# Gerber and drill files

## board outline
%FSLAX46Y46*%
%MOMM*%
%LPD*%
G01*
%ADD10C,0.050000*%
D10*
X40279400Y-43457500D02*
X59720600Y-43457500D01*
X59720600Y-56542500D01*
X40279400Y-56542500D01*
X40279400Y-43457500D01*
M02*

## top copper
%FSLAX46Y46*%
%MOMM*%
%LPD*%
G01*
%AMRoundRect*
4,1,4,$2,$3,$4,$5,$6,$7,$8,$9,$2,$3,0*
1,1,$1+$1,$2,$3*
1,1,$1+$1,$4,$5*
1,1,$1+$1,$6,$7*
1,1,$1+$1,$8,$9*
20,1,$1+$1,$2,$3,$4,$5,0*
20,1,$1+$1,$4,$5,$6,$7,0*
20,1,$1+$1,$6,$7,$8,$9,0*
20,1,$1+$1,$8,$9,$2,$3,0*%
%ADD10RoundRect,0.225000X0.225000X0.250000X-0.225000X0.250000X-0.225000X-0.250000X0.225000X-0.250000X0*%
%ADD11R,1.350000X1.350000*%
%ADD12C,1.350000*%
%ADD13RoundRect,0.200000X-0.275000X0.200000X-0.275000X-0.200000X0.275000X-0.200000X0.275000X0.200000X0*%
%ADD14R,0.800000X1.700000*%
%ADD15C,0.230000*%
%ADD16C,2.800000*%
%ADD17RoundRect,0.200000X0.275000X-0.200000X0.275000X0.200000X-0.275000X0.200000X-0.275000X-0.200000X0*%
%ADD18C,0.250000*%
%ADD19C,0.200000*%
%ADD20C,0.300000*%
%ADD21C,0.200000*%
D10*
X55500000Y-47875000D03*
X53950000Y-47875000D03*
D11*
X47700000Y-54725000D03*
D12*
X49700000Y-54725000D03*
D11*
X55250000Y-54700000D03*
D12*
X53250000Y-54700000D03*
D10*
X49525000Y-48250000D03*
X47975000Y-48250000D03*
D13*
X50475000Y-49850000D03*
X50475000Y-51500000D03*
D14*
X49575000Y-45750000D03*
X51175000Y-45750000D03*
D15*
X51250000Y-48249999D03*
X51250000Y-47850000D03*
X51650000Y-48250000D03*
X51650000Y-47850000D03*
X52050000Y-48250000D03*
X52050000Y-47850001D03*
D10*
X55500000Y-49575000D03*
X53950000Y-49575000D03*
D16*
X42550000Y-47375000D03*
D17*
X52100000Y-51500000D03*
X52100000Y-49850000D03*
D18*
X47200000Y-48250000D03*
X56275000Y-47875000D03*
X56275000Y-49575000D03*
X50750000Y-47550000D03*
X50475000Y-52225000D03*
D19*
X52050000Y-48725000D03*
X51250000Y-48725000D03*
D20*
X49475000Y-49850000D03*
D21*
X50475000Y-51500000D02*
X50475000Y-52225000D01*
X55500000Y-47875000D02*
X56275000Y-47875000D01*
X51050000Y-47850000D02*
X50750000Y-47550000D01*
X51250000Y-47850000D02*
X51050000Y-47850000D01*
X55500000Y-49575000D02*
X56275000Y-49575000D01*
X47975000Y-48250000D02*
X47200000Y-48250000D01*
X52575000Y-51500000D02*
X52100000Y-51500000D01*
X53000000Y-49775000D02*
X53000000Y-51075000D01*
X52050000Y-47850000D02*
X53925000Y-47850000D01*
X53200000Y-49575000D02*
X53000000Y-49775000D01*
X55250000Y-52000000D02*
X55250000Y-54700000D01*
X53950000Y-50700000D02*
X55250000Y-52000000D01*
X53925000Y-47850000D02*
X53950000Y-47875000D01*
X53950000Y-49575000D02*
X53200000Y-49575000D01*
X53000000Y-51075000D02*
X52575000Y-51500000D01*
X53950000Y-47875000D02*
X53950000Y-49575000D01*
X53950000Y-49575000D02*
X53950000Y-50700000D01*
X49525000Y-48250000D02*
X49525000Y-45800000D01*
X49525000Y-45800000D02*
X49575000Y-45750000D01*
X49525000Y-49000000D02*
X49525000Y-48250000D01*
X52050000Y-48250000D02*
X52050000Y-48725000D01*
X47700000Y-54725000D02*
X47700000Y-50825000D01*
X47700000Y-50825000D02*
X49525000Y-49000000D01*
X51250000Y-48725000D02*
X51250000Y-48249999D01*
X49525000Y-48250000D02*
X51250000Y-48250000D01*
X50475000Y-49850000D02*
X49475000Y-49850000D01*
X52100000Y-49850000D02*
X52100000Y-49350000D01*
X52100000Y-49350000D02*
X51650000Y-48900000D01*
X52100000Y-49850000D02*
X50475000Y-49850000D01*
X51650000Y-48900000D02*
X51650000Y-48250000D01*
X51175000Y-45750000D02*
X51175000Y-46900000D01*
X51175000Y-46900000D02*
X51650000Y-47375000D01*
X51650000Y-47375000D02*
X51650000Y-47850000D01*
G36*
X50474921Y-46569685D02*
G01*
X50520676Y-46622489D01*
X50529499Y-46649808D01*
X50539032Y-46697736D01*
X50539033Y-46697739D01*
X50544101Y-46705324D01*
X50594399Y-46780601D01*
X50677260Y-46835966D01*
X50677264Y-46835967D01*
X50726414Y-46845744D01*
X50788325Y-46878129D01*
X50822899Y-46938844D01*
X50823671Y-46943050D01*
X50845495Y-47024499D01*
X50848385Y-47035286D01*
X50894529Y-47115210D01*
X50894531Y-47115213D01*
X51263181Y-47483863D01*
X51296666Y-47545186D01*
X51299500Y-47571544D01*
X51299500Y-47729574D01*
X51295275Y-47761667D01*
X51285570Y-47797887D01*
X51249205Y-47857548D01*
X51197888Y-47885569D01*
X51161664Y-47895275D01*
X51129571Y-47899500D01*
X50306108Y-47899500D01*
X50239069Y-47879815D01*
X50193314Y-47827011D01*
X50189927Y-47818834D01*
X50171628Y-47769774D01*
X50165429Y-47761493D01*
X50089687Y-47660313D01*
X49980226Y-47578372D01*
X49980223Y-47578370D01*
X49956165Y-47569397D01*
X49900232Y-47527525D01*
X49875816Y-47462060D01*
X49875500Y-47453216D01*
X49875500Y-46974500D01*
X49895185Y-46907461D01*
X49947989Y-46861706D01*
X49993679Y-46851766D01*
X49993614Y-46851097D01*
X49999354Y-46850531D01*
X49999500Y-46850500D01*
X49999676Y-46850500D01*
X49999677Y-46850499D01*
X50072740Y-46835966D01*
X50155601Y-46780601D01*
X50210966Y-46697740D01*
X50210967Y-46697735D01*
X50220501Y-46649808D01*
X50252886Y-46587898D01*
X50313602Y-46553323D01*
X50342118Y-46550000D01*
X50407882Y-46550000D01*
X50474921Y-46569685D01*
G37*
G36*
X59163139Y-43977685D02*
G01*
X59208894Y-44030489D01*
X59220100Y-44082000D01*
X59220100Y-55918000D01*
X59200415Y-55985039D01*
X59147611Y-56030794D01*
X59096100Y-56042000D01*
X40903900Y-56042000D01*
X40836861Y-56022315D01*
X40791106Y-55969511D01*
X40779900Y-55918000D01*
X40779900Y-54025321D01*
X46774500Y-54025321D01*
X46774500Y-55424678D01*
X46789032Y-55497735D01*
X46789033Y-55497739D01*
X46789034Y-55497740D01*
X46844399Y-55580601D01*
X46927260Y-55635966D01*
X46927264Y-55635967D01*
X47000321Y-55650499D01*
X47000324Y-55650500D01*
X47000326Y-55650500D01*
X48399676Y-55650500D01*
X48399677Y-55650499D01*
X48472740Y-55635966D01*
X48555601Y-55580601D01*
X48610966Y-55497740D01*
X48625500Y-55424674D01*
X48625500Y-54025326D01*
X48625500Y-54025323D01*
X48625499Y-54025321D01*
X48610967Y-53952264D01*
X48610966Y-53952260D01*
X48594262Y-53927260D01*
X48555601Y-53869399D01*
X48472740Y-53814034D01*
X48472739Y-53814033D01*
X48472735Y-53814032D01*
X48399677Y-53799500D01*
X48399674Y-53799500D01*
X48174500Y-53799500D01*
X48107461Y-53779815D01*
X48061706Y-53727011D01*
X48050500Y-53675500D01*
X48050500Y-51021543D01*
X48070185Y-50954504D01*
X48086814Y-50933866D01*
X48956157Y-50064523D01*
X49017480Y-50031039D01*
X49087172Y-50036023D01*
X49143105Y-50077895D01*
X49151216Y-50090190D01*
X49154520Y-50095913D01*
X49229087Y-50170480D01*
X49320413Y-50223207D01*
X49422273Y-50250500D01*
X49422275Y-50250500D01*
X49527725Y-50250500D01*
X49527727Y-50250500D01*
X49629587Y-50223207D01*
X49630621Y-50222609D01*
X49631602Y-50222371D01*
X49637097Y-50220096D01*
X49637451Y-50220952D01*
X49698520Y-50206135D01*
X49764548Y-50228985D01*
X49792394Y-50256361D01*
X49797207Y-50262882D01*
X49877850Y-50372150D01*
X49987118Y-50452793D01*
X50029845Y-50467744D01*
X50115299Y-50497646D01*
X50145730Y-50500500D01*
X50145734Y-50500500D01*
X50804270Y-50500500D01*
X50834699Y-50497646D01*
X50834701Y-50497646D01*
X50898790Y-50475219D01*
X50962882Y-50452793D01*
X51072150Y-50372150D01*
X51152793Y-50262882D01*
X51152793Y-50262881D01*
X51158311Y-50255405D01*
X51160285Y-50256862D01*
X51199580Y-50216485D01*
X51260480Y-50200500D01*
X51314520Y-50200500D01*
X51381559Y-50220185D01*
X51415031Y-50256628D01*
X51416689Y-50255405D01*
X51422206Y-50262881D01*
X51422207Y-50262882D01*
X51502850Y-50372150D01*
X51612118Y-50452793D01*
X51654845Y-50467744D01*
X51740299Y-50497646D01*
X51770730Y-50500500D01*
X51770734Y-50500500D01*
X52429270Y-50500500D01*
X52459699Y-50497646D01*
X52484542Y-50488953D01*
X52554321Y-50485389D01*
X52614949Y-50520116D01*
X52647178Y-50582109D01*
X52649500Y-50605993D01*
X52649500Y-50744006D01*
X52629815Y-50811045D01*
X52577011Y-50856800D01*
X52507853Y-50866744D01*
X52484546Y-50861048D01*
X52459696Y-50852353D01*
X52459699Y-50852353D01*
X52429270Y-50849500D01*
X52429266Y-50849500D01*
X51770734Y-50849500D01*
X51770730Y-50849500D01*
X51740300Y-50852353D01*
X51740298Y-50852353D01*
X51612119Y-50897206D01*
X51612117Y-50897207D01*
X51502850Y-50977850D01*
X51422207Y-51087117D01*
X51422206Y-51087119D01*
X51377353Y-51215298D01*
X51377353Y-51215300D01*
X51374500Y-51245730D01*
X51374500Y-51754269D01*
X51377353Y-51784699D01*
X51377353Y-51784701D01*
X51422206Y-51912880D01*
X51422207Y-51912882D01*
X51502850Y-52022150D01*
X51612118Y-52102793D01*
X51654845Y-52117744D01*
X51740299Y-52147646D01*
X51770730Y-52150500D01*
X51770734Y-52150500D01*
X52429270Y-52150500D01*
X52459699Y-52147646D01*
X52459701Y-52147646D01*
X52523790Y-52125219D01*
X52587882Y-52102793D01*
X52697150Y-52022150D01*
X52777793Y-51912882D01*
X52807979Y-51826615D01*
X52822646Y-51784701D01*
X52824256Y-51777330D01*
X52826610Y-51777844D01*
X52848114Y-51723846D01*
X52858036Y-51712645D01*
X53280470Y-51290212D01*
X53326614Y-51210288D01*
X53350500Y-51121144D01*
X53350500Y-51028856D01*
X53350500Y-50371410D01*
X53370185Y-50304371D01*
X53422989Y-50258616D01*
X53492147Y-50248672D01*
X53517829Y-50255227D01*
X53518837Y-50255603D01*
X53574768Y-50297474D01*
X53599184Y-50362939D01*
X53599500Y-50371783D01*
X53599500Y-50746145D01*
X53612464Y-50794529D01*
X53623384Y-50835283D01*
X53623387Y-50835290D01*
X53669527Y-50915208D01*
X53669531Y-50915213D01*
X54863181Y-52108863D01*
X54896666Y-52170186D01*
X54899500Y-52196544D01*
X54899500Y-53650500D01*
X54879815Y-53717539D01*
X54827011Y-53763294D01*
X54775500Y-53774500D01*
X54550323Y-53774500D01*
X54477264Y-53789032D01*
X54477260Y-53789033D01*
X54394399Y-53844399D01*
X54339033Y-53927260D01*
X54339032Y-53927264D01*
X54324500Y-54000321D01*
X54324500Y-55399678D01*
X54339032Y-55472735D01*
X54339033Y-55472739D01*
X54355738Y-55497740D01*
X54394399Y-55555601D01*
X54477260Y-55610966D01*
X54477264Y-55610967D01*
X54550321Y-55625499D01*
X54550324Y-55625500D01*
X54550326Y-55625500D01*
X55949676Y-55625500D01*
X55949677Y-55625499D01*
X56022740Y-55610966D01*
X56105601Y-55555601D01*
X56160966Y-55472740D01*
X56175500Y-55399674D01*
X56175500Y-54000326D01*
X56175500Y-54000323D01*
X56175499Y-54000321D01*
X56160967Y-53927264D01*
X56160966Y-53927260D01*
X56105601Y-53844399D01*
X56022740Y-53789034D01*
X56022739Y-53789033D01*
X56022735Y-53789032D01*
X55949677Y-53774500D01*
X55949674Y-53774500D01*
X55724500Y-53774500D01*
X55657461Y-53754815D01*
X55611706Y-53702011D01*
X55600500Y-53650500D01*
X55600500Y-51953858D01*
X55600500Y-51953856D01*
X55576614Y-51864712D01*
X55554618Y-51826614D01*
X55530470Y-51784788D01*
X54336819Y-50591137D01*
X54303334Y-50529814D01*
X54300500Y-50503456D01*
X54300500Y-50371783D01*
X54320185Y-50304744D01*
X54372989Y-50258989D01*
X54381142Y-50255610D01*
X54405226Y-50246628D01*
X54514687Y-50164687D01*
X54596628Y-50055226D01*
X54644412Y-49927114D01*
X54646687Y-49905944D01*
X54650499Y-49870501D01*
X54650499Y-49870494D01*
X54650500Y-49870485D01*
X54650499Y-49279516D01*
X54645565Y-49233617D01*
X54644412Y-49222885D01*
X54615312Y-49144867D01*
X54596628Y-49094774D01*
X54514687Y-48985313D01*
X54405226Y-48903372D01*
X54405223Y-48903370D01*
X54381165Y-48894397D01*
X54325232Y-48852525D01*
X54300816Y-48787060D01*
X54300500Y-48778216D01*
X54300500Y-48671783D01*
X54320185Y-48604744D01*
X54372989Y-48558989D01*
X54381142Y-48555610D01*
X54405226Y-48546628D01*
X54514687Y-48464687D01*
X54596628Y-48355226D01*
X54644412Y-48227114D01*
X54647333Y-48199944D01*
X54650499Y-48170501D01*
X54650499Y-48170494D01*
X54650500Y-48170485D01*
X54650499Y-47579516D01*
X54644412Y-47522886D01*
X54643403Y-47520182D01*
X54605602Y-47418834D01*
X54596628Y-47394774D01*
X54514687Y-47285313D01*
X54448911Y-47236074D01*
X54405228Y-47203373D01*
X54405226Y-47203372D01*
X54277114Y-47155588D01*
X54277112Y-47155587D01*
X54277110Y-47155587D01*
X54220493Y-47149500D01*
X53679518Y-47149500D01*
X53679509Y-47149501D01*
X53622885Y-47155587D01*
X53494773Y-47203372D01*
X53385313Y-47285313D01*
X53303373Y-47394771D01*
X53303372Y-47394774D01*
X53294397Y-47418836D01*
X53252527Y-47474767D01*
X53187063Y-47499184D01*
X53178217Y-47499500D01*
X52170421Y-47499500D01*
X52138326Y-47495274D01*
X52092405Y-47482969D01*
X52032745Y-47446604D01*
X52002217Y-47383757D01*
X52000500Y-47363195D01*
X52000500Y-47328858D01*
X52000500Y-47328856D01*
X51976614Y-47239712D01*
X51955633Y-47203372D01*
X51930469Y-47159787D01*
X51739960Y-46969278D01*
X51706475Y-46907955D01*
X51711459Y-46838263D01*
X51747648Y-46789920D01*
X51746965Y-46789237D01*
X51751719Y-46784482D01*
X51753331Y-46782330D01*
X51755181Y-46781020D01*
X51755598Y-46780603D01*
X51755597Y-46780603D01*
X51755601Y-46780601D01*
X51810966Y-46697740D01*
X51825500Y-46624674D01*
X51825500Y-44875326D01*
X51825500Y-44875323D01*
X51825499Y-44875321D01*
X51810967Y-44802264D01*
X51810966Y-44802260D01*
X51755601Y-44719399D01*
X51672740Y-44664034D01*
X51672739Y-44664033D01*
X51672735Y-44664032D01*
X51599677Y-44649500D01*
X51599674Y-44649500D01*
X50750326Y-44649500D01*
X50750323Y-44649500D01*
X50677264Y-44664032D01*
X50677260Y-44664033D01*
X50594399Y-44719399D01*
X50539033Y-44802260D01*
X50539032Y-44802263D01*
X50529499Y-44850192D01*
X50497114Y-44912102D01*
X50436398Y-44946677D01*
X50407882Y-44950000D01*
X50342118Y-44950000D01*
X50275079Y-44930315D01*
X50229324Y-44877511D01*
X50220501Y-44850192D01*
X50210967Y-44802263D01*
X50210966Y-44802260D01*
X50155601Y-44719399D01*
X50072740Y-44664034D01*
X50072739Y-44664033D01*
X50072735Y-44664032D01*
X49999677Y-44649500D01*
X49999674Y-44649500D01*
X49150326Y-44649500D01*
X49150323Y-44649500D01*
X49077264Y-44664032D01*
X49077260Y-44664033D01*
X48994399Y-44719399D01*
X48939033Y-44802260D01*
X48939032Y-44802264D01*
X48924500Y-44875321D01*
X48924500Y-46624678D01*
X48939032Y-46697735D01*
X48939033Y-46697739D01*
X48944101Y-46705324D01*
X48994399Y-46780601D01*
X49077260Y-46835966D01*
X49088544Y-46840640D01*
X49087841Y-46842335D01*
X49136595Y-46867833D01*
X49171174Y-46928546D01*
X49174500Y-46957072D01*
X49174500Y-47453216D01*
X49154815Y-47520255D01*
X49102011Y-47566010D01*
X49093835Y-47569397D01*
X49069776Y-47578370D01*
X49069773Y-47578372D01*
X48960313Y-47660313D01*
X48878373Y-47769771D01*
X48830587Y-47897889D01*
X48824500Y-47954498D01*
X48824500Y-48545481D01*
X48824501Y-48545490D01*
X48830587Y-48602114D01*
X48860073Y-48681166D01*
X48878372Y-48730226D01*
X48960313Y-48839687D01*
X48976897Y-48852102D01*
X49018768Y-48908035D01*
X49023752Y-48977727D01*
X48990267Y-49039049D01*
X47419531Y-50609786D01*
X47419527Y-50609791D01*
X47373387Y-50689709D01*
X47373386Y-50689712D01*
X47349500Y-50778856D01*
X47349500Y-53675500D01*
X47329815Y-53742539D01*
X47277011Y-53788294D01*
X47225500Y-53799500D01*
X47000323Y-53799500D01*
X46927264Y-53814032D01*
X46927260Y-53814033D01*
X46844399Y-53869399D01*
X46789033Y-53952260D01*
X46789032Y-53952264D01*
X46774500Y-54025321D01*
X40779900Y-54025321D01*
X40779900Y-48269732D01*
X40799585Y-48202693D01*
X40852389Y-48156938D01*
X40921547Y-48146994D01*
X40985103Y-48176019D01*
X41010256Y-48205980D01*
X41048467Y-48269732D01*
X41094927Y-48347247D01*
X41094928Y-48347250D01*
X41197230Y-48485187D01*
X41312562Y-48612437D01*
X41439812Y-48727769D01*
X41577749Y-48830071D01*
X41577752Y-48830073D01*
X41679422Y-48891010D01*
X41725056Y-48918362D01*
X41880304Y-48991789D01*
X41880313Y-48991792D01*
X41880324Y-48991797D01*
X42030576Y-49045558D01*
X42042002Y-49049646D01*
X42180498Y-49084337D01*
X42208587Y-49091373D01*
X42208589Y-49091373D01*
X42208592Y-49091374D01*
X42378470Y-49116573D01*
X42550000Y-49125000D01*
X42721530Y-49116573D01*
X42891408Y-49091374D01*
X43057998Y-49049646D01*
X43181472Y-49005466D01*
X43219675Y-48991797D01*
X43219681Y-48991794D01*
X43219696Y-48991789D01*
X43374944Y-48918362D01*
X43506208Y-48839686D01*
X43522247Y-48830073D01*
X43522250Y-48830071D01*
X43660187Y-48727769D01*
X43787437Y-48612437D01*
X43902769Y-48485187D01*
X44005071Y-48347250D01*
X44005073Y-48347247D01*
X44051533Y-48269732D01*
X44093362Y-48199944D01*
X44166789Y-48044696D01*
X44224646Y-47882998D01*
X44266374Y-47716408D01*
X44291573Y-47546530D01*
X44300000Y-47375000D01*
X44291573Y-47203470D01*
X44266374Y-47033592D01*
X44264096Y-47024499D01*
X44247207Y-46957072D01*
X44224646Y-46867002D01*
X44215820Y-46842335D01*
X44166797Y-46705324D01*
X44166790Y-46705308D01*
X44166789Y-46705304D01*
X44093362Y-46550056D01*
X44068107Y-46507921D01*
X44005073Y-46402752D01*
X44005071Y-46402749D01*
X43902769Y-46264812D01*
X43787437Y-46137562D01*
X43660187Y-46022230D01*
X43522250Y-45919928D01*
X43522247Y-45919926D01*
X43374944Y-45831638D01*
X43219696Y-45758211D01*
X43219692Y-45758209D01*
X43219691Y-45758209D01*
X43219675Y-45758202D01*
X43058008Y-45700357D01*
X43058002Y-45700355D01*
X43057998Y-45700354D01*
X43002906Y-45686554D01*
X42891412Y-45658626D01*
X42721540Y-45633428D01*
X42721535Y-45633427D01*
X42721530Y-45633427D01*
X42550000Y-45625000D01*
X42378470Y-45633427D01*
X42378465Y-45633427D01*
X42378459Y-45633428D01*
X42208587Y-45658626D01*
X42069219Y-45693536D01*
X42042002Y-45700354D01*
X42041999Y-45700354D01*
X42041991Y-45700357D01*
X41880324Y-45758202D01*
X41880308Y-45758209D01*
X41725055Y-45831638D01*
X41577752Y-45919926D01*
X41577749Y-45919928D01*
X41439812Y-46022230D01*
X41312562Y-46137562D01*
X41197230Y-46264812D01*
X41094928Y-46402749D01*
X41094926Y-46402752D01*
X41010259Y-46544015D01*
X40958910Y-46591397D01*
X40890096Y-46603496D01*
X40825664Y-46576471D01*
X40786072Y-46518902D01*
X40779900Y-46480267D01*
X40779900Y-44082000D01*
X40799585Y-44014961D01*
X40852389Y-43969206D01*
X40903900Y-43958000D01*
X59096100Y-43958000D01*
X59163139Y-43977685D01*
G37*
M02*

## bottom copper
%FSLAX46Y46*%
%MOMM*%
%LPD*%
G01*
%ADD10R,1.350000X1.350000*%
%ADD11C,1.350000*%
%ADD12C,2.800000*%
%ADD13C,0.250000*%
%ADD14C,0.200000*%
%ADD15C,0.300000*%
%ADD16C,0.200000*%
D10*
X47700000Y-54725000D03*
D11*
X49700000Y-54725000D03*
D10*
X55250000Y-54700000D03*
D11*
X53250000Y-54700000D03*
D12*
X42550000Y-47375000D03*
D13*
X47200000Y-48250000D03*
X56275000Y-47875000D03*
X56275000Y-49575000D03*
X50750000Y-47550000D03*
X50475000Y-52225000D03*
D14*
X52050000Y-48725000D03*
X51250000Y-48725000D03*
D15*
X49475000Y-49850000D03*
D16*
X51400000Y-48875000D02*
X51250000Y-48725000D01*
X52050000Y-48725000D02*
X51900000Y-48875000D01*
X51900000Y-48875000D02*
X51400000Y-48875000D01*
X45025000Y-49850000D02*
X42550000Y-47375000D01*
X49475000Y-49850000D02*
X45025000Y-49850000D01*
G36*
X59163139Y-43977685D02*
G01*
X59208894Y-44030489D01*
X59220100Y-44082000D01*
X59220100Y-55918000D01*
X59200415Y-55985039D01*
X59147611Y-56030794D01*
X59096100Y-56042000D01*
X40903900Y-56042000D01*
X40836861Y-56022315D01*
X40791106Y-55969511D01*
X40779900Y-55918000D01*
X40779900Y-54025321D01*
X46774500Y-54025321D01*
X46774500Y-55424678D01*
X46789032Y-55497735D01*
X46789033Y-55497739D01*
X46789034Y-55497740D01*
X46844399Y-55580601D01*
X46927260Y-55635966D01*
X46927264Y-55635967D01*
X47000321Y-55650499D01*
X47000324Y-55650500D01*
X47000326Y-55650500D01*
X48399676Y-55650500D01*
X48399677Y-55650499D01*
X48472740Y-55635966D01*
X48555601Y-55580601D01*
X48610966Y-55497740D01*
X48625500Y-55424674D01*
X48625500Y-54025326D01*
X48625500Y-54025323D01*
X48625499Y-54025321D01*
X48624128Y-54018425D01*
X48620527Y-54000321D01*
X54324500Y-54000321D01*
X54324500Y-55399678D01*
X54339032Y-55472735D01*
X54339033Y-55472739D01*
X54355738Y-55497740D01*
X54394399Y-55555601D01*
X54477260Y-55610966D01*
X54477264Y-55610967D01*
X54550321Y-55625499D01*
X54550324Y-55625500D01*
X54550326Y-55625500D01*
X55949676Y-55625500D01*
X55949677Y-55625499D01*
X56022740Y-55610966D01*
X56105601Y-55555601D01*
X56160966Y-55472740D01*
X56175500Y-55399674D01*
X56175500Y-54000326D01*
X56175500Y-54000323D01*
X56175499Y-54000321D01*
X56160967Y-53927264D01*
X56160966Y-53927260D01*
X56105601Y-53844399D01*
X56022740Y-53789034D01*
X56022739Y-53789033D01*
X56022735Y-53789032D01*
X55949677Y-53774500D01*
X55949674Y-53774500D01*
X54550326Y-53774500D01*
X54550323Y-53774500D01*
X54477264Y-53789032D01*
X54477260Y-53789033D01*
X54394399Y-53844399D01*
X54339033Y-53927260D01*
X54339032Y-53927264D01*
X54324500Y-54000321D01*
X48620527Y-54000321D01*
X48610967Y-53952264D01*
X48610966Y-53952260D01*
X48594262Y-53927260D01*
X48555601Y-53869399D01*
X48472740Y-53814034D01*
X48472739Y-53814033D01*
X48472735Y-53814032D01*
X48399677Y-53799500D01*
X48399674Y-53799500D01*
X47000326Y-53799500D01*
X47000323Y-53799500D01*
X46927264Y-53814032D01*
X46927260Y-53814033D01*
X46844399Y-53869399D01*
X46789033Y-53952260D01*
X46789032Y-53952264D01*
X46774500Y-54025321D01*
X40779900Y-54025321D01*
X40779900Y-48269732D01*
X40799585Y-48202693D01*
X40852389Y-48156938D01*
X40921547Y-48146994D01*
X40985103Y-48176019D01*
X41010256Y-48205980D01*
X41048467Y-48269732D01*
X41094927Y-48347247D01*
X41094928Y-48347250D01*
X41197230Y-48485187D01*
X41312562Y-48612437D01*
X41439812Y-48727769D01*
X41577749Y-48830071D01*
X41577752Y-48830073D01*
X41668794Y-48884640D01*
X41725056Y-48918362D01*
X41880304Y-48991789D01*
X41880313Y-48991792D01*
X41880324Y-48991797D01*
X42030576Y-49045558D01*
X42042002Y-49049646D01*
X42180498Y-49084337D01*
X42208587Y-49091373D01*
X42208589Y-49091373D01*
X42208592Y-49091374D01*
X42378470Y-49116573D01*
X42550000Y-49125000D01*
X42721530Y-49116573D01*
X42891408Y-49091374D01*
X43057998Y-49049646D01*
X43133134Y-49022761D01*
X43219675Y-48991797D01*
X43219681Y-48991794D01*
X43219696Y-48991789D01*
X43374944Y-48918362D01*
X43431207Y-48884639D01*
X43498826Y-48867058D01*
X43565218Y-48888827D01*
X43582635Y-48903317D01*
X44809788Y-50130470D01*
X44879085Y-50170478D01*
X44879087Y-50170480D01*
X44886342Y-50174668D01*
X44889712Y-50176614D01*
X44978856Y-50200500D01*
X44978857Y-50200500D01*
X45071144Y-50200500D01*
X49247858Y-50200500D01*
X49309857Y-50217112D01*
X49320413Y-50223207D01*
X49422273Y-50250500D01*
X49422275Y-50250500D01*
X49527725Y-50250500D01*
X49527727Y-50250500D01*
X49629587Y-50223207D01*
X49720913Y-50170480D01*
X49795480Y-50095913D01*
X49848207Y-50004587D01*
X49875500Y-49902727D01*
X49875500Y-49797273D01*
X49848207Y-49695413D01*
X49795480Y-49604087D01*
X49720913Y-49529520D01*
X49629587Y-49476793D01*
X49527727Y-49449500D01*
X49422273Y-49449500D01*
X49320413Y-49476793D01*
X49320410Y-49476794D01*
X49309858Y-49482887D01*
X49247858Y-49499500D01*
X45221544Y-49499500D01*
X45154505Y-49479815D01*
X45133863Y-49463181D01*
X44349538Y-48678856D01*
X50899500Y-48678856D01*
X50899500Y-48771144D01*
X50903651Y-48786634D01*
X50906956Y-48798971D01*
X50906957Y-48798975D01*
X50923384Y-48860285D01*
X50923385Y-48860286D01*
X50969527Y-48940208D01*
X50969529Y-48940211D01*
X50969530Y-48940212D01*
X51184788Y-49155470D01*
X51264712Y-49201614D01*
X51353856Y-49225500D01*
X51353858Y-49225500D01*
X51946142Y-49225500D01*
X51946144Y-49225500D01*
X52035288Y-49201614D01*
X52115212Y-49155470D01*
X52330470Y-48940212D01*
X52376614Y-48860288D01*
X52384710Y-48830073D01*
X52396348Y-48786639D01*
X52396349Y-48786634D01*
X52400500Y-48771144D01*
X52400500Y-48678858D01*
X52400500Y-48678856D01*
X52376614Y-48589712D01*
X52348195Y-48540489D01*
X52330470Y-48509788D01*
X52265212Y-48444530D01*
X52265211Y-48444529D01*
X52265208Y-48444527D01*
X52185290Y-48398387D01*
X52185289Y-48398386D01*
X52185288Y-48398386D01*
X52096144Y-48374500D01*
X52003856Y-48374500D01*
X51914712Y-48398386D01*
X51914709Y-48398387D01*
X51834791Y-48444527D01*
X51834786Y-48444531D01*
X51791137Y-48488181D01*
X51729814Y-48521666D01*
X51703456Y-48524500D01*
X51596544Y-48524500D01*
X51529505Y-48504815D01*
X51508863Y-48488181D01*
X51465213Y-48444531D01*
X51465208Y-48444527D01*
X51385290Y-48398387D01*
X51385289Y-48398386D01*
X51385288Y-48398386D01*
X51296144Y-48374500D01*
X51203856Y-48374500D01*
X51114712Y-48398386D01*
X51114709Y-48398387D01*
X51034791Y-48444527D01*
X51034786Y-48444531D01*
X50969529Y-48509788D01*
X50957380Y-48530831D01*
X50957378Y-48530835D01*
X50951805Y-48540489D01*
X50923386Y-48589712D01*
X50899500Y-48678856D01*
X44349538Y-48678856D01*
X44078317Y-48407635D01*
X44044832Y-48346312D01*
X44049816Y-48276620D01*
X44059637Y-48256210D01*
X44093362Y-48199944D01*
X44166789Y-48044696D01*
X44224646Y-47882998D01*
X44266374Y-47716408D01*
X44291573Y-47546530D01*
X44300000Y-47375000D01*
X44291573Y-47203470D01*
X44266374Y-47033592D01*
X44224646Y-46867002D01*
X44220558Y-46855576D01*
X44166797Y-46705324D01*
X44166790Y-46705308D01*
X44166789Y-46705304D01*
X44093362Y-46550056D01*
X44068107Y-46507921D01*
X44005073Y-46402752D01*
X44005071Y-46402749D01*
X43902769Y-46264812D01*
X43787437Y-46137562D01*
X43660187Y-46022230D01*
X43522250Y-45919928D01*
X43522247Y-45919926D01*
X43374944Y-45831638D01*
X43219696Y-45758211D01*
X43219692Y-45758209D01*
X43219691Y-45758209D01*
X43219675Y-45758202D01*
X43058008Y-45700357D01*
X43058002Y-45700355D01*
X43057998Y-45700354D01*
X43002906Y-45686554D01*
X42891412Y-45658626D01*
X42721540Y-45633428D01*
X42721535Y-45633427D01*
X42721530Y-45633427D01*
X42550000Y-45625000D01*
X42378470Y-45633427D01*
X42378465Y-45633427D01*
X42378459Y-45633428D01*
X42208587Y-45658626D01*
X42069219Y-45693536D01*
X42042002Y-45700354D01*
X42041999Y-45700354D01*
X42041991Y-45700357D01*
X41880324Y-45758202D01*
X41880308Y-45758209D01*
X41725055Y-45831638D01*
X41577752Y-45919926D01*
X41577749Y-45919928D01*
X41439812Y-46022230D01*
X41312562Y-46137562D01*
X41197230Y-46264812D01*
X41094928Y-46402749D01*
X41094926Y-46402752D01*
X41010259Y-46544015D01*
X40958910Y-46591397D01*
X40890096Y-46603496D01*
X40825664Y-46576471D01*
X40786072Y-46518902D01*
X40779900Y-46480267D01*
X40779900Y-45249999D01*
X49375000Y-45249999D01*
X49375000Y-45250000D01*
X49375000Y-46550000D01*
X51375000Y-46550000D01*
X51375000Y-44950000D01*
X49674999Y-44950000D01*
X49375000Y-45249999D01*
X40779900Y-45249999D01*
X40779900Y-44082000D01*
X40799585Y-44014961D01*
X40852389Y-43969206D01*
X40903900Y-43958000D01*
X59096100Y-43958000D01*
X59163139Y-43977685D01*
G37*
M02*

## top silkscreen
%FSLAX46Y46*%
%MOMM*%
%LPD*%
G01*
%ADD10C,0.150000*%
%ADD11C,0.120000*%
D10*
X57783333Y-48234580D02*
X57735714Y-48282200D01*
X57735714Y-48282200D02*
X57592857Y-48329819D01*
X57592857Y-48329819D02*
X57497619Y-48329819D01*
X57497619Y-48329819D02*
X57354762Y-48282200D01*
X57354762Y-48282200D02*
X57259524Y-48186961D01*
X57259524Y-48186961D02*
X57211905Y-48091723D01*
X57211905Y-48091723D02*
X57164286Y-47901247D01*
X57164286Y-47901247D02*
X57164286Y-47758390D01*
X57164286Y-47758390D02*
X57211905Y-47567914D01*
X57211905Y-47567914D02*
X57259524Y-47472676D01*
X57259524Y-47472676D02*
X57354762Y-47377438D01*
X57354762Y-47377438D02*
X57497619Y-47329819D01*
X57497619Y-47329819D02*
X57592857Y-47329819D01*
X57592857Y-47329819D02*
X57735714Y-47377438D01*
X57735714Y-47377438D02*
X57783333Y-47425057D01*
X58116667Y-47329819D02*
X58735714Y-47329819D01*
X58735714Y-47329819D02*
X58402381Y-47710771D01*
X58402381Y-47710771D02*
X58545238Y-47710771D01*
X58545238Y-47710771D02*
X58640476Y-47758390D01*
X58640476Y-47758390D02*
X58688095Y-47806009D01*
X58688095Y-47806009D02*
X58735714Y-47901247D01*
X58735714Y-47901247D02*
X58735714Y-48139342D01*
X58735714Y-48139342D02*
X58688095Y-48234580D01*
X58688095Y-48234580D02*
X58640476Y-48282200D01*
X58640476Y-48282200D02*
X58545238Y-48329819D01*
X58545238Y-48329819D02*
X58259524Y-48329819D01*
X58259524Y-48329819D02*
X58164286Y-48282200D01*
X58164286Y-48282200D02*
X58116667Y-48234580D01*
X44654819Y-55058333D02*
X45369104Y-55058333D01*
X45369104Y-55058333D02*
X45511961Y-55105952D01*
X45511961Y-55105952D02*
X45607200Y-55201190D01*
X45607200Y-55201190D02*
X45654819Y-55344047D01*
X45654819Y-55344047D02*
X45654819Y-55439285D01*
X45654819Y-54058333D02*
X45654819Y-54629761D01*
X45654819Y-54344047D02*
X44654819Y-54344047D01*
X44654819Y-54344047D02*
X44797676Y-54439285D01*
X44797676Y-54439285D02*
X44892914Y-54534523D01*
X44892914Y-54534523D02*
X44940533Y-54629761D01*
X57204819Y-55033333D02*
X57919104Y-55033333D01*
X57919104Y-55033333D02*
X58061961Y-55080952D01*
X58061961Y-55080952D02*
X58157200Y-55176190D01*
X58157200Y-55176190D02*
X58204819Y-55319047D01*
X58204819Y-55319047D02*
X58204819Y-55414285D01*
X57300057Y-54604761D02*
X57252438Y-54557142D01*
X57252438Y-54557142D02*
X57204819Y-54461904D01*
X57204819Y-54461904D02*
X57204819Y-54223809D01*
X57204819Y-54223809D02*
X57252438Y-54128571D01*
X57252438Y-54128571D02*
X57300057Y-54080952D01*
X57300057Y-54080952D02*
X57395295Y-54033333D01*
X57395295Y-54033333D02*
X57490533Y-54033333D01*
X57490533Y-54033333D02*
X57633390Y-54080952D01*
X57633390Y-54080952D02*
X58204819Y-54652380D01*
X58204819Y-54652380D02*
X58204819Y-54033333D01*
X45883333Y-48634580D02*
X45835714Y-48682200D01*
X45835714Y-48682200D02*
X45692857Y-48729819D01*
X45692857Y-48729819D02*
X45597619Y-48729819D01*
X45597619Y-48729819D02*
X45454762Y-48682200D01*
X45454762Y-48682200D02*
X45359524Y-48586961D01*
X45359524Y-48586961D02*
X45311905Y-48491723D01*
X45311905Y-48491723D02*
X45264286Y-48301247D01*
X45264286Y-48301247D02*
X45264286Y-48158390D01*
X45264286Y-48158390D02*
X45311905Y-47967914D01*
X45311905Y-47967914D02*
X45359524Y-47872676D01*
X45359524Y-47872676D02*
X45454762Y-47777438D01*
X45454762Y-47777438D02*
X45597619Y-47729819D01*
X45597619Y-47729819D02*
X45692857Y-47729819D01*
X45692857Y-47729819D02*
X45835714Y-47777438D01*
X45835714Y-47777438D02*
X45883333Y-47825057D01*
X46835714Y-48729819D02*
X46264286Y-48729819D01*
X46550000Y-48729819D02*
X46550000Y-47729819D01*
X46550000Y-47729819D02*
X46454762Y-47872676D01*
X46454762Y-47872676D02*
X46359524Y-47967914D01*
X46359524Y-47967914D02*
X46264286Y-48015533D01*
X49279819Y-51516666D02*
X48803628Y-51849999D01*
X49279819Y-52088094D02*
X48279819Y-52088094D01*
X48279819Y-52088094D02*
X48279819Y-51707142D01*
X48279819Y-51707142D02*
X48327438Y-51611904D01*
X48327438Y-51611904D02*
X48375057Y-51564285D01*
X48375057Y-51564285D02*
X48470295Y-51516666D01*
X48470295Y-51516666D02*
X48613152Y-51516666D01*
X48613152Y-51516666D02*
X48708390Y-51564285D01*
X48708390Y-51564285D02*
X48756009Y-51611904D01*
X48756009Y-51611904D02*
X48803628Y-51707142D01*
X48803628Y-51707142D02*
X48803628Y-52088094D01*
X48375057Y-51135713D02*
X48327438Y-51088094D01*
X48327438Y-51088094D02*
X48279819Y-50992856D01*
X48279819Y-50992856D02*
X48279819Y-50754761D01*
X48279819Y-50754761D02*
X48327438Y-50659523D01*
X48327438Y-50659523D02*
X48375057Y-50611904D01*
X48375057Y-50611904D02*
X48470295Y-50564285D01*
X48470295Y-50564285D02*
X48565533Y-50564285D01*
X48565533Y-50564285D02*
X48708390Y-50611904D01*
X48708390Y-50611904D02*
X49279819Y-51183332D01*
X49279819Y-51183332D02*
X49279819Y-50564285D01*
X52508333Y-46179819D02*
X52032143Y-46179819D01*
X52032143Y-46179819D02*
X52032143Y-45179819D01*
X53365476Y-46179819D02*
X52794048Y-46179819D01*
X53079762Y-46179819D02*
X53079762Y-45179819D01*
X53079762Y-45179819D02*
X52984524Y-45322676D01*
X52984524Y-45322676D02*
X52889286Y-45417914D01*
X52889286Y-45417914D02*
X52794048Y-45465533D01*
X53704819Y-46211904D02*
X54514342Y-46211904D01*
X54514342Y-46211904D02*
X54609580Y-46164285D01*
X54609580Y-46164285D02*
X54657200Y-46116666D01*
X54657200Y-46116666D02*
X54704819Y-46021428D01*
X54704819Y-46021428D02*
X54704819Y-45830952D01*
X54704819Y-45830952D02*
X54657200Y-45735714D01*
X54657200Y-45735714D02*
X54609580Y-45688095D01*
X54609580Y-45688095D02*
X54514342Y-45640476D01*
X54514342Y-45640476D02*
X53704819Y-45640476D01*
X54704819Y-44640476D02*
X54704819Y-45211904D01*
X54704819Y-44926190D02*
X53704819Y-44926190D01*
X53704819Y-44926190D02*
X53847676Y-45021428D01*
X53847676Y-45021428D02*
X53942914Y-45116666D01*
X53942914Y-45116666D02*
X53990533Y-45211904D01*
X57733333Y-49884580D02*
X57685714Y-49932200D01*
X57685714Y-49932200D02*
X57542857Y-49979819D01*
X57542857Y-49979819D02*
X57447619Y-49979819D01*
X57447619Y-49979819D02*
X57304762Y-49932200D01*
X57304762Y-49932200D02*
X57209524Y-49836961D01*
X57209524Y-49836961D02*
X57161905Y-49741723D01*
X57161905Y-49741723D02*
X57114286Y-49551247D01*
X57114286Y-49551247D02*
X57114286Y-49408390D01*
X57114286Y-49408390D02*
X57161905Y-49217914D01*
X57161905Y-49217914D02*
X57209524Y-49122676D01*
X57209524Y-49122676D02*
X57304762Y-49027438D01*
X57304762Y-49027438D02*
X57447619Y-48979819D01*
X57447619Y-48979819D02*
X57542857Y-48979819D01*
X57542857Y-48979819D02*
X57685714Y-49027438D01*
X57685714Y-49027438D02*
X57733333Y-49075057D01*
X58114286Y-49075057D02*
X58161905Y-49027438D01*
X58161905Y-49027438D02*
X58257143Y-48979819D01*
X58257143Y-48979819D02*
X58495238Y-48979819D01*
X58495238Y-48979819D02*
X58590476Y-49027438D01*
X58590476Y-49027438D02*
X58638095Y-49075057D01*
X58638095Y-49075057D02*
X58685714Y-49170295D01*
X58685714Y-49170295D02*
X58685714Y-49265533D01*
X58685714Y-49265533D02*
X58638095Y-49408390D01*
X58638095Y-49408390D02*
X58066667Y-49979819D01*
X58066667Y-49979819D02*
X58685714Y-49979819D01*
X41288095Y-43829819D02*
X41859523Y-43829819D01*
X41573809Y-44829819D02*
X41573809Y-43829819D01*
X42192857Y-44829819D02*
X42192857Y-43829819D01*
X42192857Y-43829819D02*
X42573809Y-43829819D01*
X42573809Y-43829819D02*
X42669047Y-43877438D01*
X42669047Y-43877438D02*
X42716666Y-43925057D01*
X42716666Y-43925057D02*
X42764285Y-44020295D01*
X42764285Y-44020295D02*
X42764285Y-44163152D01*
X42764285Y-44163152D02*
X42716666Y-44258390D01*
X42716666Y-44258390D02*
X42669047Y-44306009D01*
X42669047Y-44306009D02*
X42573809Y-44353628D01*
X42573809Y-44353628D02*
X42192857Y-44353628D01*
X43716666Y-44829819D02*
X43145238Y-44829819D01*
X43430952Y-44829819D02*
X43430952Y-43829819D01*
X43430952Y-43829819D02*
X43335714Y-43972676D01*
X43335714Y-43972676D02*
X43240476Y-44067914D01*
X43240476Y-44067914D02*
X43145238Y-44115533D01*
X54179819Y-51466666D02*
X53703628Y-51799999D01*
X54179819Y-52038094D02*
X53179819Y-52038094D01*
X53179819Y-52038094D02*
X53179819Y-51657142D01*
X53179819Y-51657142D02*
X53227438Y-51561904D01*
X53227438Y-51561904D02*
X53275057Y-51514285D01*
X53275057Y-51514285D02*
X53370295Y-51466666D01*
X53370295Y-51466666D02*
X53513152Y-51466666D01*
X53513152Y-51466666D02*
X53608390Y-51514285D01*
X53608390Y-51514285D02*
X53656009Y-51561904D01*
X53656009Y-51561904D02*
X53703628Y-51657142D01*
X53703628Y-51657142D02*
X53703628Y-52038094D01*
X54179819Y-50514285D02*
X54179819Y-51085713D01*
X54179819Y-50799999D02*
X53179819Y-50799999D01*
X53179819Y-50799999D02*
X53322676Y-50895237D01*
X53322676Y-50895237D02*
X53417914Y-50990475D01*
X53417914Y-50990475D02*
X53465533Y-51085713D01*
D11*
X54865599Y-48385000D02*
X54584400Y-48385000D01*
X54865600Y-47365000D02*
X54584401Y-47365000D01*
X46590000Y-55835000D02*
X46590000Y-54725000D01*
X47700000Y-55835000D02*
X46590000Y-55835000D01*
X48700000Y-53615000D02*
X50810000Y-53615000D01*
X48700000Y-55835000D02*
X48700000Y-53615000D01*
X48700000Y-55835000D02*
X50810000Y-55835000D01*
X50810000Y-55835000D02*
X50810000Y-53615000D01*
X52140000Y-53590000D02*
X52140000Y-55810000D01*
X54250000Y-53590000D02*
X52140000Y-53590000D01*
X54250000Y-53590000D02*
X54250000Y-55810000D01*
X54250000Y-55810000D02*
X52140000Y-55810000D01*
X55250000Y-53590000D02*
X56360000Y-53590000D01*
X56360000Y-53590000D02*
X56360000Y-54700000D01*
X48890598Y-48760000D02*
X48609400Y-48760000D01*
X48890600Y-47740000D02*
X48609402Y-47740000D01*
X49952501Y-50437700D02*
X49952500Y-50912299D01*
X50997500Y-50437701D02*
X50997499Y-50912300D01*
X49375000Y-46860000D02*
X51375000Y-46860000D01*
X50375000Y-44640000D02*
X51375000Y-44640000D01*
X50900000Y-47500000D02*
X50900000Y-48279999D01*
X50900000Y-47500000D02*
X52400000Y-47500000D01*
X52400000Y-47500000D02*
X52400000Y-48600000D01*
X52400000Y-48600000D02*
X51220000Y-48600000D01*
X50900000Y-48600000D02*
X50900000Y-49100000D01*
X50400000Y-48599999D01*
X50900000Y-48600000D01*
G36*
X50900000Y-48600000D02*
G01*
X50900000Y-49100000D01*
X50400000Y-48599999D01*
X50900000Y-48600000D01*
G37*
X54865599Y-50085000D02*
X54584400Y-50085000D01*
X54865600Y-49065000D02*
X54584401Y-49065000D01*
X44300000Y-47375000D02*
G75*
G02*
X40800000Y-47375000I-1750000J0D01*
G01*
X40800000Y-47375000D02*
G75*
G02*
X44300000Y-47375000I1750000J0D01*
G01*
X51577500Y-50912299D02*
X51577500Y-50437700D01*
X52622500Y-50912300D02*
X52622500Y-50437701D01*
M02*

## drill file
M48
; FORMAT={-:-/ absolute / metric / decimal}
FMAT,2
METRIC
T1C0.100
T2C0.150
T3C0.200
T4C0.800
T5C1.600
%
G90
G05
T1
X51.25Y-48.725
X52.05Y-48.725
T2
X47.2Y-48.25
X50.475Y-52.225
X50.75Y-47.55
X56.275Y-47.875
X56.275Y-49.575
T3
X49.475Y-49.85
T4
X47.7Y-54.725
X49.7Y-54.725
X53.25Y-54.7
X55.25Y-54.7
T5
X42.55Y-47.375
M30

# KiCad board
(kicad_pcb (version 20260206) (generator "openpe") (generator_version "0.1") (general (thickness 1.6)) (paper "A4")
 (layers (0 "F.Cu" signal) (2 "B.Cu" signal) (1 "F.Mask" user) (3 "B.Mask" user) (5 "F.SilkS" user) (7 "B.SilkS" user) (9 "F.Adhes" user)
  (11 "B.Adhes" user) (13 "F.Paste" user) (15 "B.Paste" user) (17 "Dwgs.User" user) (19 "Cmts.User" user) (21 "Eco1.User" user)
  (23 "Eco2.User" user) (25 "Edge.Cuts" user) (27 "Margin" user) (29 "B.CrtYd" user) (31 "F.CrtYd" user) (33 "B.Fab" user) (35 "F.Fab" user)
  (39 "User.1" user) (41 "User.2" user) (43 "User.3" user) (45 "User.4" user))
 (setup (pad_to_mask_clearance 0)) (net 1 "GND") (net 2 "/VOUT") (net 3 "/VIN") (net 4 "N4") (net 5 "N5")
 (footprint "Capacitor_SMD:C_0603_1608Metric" (layer "F.Cu") (at 54.725 47.875 180)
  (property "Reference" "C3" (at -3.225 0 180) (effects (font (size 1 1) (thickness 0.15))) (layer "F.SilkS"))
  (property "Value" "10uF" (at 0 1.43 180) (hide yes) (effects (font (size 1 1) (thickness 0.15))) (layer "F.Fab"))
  (fp_line (start -0.140599 -0.51) (end 0.1406 -0.51) (stroke (width 0.12) (type solid)) (layer "F.SilkS"))
  (fp_line (start -0.1406 0.51) (end 0.140599 0.51) (stroke (width 0.12) (type solid)) (layer "F.SilkS"))
  (pad "1" smd roundrect (at -0.775 0 180) (size 0.9 0.95) (layers "F.Cu" "F.Mask" "F.Paste") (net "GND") (roundrect_rratio 0.25))
  (pad "2" smd roundrect (at 0.775 0 180) (size 0.9 0.95) (layers "F.Cu" "F.Mask" "F.Paste") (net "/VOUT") (roundrect_rratio 0.25)))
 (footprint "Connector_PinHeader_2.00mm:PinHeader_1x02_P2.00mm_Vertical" (layer "F.Cu") (at 48.7 54.725 90)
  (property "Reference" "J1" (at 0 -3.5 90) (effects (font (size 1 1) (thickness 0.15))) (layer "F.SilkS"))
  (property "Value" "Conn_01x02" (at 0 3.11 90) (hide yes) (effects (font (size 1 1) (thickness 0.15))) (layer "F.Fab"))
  (fp_line (start -1.11 -2.11) (end 0 -2.11) (stroke (width 0.12) (type solid)) (layer "F.SilkS"))
  (fp_line (start -1.11 -1) (end -1.11 -2.11) (stroke (width 0.12) (type solid)) (layer "F.SilkS"))
  (fp_line (start 1.11 0) (end 1.11 2.11) (stroke (width 0.12) (type solid)) (layer "F.SilkS"))
  (fp_line (start -1.11 0) (end 1.11 0) (stroke (width 0.12) (type solid)) (layer "F.SilkS"))
  (fp_line (start -1.11 0) (end -1.11 2.11) (stroke (width 0.12) (type solid)) (layer "F.SilkS"))
  (fp_line (start -1.11 2.11) (end 1.11 2.11) (stroke (width 0.12) (type solid)) (layer "F.SilkS"))
  (pad "1" thru_hole rect (at 0 -1 90) (size 1.35 1.35) (drill 0.8) (layers "*.Cu" "*.Mask") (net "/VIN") (remove_unused_layers no))
  (pad "2" thru_hole circle (at 0 1 90) (size 1.35 1.35) (drill 0.8) (layers "*.Cu" "*.Mask") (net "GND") (remove_unused_layers no)))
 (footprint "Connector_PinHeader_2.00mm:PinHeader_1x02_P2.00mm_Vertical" (layer "F.Cu") (at 54.25 54.7 -90)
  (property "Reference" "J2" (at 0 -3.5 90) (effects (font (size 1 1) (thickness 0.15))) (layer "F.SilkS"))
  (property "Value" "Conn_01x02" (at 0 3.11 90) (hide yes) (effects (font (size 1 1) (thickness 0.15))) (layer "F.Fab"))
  (fp_line (start -1.11 2.11) (end 1.11 2.11) (stroke (width 0.12) (type solid)) (layer "F.SilkS"))
  (fp_line (start -1.11 0) (end -1.11 2.11) (stroke (width 0.12) (type solid)) (layer "F.SilkS"))
  (fp_line (start -1.11 0) (end 1.11 0) (stroke (width 0.12) (type solid)) (layer "F.SilkS"))
  (fp_line (start 1.11 0) (end 1.11 2.11) (stroke (width 0.12) (type solid)) (layer "F.SilkS"))
  (fp_line (start -1.11 -1) (end -1.11 -2.11) (stroke (width 0.12) (type solid)) (layer "F.SilkS"))
  (fp_line (start -1.11 -2.11) (end 0 -2.11) (stroke (width 0.12) (type solid)) (layer "F.SilkS"))
  (pad "1" thru_hole rect (at 0 -1 -90) (size 1.35 1.35) (drill 0.8) (layers "*.Cu" "*.Mask") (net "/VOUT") (remove_unused_layers no))
  (pad "2" thru_hole circle (at 0 1 -90) (size 1.35 1.35) (drill 0.8) (layers "*.Cu" "*.Mask") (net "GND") (remove_unused_layers no)))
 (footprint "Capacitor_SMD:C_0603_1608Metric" (layer "F.Cu") (at 48.75 48.25 180)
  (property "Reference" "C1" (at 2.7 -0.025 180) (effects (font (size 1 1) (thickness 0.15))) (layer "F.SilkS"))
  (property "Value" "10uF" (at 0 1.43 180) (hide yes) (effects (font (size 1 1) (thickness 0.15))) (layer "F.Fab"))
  (fp_line (start -0.140598 -0.51) (end 0.1406 -0.51) (stroke (width 0.12) (type solid)) (layer "F.SilkS"))
  (fp_line (start -0.1406 0.51) (end 0.140598 0.51) (stroke (width 0.12) (type solid)) (layer "F.SilkS"))
  (pad "1" smd roundrect (at -0.775 0 180) (size 0.9 0.95) (layers "F.Cu" "F.Mask" "F.Paste") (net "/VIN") (roundrect_rratio 0.25))
  (pad "2" smd roundrect (at 0.775 0 180) (size 0.9 0.95) (layers "F.Cu" "F.Mask" "F.Paste") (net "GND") (roundrect_rratio 0.25)))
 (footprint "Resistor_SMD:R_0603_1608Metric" (layer "F.Cu") (at 50.475 50.675 -90)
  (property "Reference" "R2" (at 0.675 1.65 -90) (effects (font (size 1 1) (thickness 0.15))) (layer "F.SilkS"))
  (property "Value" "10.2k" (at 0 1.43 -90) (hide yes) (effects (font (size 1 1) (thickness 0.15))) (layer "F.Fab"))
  (fp_line (start -0.2373 0.522499) (end 0.237299 0.5225) (stroke (width 0.12) (type solid)) (layer "F.SilkS"))
  (fp_line (start -0.237299 -0.5225) (end 0.2373 -0.522499) (stroke (width 0.12) (type solid)) (layer "F.SilkS"))
  (pad "1" smd roundrect (at -0.825 0 -90) (size 0.8 0.95) (layers "F.Cu" "F.Mask" "F.Paste") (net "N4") (roundrect_rratio 0.25))
  (pad "2" smd roundrect (at 0.825 0 -90) (size 0.8 0.95) (layers "F.Cu" "F.Mask" "F.Paste") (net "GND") (roundrect_rratio 0.25)))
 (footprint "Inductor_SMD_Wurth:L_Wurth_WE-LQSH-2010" (layer "F.Cu") (at 50.375 45.75 0)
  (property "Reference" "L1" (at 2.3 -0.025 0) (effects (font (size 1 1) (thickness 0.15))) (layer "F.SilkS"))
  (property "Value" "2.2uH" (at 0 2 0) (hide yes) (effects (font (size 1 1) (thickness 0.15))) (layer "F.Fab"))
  (fp_line (start -1 1.11) (end 1 1.11) (stroke (width 0.12) (type solid)) (layer "F.SilkS"))
  (fp_line (start 0 -1.11) (end 1 -1.11) (stroke (width 0.12) (type solid)) (layer "F.SilkS"))
  (pad "1" smd rect (at -0.8 0 0) (size 0.8 1.7) (layers "F.Cu" "F.Mask" "F.Paste") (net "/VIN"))
  (pad "2" smd rect (at 0.8 0 0) (size 0.8 1.7) (layers "F.Cu" "F.Mask" "F.Paste") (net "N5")))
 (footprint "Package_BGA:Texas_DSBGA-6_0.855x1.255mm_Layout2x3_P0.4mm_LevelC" (layer "F.Cu") (at 51.65 48.05 90)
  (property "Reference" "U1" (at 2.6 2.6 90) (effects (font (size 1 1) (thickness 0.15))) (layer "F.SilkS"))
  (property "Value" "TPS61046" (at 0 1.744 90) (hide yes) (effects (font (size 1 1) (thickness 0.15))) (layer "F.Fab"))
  (fp_line (start 0.55 -0.75) (end -0.229999 -0.75) (stroke (width 0.12) (type solid)) (layer "F.SilkS"))
  (fp_line (start 0.55 -0.75) (end 0.55 0.75) (stroke (width 0.12) (type solid)) (layer "F.SilkS"))
  (fp_line (start 0.55 0.75) (end -0.55 0.75) (stroke (width 0.12) (type solid)) (layer "F.SilkS"))
  (fp_line (start -0.55 0.75) (end -0.55 -0.43) (stroke (width 0.12) (type solid)) (layer "F.SilkS"))
  (fp_poly (pts (xy -0.55 -0.75) (xy -1.05 -0.75) (xy -0.549999 -1.25)) (stroke (width 0.12) (type solid)) (fill yes) (layer "F.SilkS"))
  (pad "A1" smd circle (at -0.199999 -0.4 90) (size 0.23 0.23) (layers "F.Cu" "F.Mask") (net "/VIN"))
  (pad "A2" smd circle (at 0.2 -0.4 90) (size 0.23 0.23) (layers "F.Cu" "F.Mask") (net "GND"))
  (pad "B1" smd circle (at -0.2 0 90) (size 0.23 0.23) (layers "F.Cu" "F.Mask") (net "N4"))
  (pad "B2" smd circle (at 0.2 0 90) (size 0.23 0.23) (layers "F.Cu" "F.Mask") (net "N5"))
  (pad "C1" smd circle (at -0.2 0.4 90) (size 0.23 0.23) (layers "F.Cu" "F.Mask") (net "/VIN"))
  (pad "C2" smd circle (at 0.199999 0.4 90) (size 0.23 0.23) (layers "F.Cu" "F.Mask") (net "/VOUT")))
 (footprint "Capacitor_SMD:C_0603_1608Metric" (layer "F.Cu") (at 54.725 49.575 180)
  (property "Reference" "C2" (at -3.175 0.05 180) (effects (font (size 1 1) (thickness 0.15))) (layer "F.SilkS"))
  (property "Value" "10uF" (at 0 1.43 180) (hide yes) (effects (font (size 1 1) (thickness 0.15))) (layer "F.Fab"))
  (fp_line (start -0.140599 -0.51) (end 0.1406 -0.51) (stroke (width 0.12) (type solid)) (layer "F.SilkS"))
  (fp_line (start -0.1406 0.51) (end 0.140599 0.51) (stroke (width 0.12) (type solid)) (layer "F.SilkS"))
  (pad "1" smd roundrect (at -0.775 0 180) (size 0.9 0.95) (layers "F.Cu" "F.Mask" "F.Paste") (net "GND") (roundrect_rratio 0.25))
  (pad "2" smd roundrect (at 0.775 0 180) (size 0.9 0.95) (layers "F.Cu" "F.Mask" "F.Paste") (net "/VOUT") (roundrect_rratio 0.25)))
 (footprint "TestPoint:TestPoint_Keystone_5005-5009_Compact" (layer "F.Cu") (at 42.55 47.375 0)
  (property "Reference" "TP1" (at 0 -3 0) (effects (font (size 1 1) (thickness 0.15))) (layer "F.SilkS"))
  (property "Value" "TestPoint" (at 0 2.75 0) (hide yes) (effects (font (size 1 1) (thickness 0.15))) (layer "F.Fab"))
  (fp_circle (center 0 0) (end 1.75 0) (stroke (width 0.12) (type solid)) (fill no) (layer "F.SilkS"))
  (pad "1" thru_hole circle (at 0 0 0) (size 2.8 2.8) (drill 1.6) (layers "*.Cu" "*.Mask") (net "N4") (remove_unused_layers no)))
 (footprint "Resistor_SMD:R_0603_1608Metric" (layer "F.Cu") (at 52.1 50.675 90)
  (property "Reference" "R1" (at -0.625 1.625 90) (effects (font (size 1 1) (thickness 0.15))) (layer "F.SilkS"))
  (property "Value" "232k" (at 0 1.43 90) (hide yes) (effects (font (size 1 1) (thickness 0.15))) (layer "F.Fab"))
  (fp_line (start -0.237299 -0.5225) (end 0.2373 -0.5225) (stroke (width 0.12) (type solid)) (layer "F.SilkS"))
  (fp_line (start -0.2373 0.5225) (end 0.237299 0.5225) (stroke (width 0.12) (type solid)) (layer "F.SilkS"))
  (pad "1" smd roundrect (at -0.825 0 90) (size 0.8 0.95) (layers "F.Cu" "F.Mask" "F.Paste") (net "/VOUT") (roundrect_rratio 0.25))
  (pad "2" smd roundrect (at 0.825 0 90) (size 0.8 0.95) (layers "F.Cu" "F.Mask" "F.Paste") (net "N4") (roundrect_rratio 0.25)))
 (gr_poly
  (pts (xy 40.2794 43.4575) (xy 59.7206 43.4575) (xy 59.7206 56.5425) (xy 40.2794 56.5425)) (stroke (width 0.05) (type solid)) (fill no)
  (layer "Edge.Cuts"))
 (segment (start 50.475 51.5) (end 50.475 52.225) (width 0.2) (layer "F.Cu") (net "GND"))
 (segment (start 55.5 47.875) (end 56.275 47.875) (width 0.2) (layer "F.Cu") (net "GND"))
 (segment (start 51.05 47.85) (end 50.75 47.55) (width 0.2) (layer "F.Cu") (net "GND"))
 (segment (start 51.25 47.85) (end 51.05 47.85) (width 0.2) (layer "F.Cu") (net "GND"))
 (segment (start 55.5 49.575) (end 56.275 49.575) (width 0.2) (layer "F.Cu") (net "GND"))
 (segment (start 47.975 48.25) (end 47.2 48.25) (width 0.2) (layer "F.Cu") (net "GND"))
 (segment (start 52.575 51.5) (end 52.1 51.5) (width 0.2) (layer "F.Cu") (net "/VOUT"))
 (segment (start 53 49.775) (end 53 51.075) (width 0.2) (layer "F.Cu") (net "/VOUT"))
 (segment (start 52.05 47.85) (end 53.925 47.85) (width 0.2) (layer "F.Cu") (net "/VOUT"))
 (segment (start 53.2 49.575) (end 53 49.775) (width 0.2) (layer "F.Cu") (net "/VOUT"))
 (segment (start 55.25 52) (end 55.25 54.7) (width 0.2) (layer "F.Cu") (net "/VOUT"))
 (segment (start 53.95 50.7) (end 55.25 52) (width 0.2) (layer "F.Cu") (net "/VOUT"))
 (segment (start 53.925 47.85) (end 53.95 47.875) (width 0.2) (layer "F.Cu") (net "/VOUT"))
 (segment (start 53.95 49.575) (end 53.2 49.575) (width 0.2) (layer "F.Cu") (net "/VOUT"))
 (segment (start 53 51.075) (end 52.575 51.5) (width 0.2) (layer "F.Cu") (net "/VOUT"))
 (segment (start 53.95 47.875) (end 53.95 49.575) (width 0.2) (layer "F.Cu") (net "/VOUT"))
 (segment (start 53.95 49.575) (end 53.95 50.7) (width 0.2) (layer "F.Cu") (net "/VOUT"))
 (segment (start 49.525 48.25) (end 49.525 45.8) (width 0.2) (layer "F.Cu") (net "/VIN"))
 (segment (start 49.525 45.8) (end 49.575 45.75) (width 0.2) (layer "F.Cu") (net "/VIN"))
 (segment (start 49.525 49) (end 49.525 48.25) (width 0.2) (layer "F.Cu") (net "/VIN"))
 (segment (start 52.05 48.25) (end 52.05 48.725) (width 0.2) (layer "F.Cu") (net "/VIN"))
 (segment (start 47.7 54.725) (end 47.7 50.825) (width 0.2) (layer "F.Cu") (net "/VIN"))
 (segment (start 47.7 50.825) (end 49.525 49) (width 0.2) (layer "F.Cu") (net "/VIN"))
 (segment (start 51.25 48.725) (end 51.25 48.249999) (width 0.2) (layer "F.Cu") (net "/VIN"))
 (segment (start 49.525 48.25) (end 51.25 48.25) (width 0.2) (layer "F.Cu") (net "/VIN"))
 (segment (start 51.4 48.875) (end 51.25 48.725) (width 0.2) (layer "B.Cu") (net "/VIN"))
 (segment (start 52.05 48.725) (end 51.9 48.875) (width 0.2) (layer "B.Cu") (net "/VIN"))
 (segment (start 51.9 48.875) (end 51.4 48.875) (width 0.2) (layer "B.Cu") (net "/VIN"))
 (segment (start 50.475 49.85) (end 49.475 49.85) (width 0.2) (layer "F.Cu") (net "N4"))
 (segment (start 52.1 49.85) (end 52.1 49.35) (width 0.2) (layer "F.Cu") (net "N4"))
 (segment (start 52.1 49.35) (end 51.65 48.9) (width 0.2) (layer "F.Cu") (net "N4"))
 (segment (start 52.1 49.85) (end 50.475 49.85) (width 0.2) (layer "F.Cu") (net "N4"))
 (segment (start 51.65 48.9) (end 51.65 48.25) (width 0.2) (layer "F.Cu") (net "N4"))
 (segment (start 45.025 49.85) (end 42.55 47.375) (width 0.2) (layer "B.Cu") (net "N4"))
 (segment (start 49.475 49.85) (end 45.025 49.85) (width 0.2) (layer "B.Cu") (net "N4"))
 (segment (start 51.175 45.75) (end 51.175 46.9) (width 0.2) (layer "F.Cu") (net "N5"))
 (segment (start 51.175 46.9) (end 51.65 47.375) (width 0.2) (layer "F.Cu") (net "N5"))
 (segment (start 51.65 47.375) (end 51.65 47.85) (width 0.2) (layer "F.Cu") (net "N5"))
 (via (at 47.2 48.25) (size 0.25) (drill 0.15) (layers "F.Cu" "B.Cu") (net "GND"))
 (via (at 56.275 47.875) (size 0.25) (drill 0.15) (layers "F.Cu" "B.Cu") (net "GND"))
 (via (at 56.275 49.575) (size 0.25) (drill 0.15) (layers "F.Cu" "B.Cu") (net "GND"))
 (via (at 50.75 47.55) (size 0.25) (drill 0.15) (layers "F.Cu" "B.Cu") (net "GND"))
 (via (at 50.475 52.225) (size 0.25) (drill 0.15) (layers "F.Cu" "B.Cu") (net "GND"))
 (via (at 52.05 48.725) (size 0.2) (drill 0.1) (layers "F.Cu" "B.Cu") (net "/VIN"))
 (via (at 51.25 48.725) (size 0.2) (drill 0.1) (layers "F.Cu" "B.Cu") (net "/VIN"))
 (via (at 49.475 49.85) (size 0.3) (drill 0.2) (layers "F.Cu" "B.Cu") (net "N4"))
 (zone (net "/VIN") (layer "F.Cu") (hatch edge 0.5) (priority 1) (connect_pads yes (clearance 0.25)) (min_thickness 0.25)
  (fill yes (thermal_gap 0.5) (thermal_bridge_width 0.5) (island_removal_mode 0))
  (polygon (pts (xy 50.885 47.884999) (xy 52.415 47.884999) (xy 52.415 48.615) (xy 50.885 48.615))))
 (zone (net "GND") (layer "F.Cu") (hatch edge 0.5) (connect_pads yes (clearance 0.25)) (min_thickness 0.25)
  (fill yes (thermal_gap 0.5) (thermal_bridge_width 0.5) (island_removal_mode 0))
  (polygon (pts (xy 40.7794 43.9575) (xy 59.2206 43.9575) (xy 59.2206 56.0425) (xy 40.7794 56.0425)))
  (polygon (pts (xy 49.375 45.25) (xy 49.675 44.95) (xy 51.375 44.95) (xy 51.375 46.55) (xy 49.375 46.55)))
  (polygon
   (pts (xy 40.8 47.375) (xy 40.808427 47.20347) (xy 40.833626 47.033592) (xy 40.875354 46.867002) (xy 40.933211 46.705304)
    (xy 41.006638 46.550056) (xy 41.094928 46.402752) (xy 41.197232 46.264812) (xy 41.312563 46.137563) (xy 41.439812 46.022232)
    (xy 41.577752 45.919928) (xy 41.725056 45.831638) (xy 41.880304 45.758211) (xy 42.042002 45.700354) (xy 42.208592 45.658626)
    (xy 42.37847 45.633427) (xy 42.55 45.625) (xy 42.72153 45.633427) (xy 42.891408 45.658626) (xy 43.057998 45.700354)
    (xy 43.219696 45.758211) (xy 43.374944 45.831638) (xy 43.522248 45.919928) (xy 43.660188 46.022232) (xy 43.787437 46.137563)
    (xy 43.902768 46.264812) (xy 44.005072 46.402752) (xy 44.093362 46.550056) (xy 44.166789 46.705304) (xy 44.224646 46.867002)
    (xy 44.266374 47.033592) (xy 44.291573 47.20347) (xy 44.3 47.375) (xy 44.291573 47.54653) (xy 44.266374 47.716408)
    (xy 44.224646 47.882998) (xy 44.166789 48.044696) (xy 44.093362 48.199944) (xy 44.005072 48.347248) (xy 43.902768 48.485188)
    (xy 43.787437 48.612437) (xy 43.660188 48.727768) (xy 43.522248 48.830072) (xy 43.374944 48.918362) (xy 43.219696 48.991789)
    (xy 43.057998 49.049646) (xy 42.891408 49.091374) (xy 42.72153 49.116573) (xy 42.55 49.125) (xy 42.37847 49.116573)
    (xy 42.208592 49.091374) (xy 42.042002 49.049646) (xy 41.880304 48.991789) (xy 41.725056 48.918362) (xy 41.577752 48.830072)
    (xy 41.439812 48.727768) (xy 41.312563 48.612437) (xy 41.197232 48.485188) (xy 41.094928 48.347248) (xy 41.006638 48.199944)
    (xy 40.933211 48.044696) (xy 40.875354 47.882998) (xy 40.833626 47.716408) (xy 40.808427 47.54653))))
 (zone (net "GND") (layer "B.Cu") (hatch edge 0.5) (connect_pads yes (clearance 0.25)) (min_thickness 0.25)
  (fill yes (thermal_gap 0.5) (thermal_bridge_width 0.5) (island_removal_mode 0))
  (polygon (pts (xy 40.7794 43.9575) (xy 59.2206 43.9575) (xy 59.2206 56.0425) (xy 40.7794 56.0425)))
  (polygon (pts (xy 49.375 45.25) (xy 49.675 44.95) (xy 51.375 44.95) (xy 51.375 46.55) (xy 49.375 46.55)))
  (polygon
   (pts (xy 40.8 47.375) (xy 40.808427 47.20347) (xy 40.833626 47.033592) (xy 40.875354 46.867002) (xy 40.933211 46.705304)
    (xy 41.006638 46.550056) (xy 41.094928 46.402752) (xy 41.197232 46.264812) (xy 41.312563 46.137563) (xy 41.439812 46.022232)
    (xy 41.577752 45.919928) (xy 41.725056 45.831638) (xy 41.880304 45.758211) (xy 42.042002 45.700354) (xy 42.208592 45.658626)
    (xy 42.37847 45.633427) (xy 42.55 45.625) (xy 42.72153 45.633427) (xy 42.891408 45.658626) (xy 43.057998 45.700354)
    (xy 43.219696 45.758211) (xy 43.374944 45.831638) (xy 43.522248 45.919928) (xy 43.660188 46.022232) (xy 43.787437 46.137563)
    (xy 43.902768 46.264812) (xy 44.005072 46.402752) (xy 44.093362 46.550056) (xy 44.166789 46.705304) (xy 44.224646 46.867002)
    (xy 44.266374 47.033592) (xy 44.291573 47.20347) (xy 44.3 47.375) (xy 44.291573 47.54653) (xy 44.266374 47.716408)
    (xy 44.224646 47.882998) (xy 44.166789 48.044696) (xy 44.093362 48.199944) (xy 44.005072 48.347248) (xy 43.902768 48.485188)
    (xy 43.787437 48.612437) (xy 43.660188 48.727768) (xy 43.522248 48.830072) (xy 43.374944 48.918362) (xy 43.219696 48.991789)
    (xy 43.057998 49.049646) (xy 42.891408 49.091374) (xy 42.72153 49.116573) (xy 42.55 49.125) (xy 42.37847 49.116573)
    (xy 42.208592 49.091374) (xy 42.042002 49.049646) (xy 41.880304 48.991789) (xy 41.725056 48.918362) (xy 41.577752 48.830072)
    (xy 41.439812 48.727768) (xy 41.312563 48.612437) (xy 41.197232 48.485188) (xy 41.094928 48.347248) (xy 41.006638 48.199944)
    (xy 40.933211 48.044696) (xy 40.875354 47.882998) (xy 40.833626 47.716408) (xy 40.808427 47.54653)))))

